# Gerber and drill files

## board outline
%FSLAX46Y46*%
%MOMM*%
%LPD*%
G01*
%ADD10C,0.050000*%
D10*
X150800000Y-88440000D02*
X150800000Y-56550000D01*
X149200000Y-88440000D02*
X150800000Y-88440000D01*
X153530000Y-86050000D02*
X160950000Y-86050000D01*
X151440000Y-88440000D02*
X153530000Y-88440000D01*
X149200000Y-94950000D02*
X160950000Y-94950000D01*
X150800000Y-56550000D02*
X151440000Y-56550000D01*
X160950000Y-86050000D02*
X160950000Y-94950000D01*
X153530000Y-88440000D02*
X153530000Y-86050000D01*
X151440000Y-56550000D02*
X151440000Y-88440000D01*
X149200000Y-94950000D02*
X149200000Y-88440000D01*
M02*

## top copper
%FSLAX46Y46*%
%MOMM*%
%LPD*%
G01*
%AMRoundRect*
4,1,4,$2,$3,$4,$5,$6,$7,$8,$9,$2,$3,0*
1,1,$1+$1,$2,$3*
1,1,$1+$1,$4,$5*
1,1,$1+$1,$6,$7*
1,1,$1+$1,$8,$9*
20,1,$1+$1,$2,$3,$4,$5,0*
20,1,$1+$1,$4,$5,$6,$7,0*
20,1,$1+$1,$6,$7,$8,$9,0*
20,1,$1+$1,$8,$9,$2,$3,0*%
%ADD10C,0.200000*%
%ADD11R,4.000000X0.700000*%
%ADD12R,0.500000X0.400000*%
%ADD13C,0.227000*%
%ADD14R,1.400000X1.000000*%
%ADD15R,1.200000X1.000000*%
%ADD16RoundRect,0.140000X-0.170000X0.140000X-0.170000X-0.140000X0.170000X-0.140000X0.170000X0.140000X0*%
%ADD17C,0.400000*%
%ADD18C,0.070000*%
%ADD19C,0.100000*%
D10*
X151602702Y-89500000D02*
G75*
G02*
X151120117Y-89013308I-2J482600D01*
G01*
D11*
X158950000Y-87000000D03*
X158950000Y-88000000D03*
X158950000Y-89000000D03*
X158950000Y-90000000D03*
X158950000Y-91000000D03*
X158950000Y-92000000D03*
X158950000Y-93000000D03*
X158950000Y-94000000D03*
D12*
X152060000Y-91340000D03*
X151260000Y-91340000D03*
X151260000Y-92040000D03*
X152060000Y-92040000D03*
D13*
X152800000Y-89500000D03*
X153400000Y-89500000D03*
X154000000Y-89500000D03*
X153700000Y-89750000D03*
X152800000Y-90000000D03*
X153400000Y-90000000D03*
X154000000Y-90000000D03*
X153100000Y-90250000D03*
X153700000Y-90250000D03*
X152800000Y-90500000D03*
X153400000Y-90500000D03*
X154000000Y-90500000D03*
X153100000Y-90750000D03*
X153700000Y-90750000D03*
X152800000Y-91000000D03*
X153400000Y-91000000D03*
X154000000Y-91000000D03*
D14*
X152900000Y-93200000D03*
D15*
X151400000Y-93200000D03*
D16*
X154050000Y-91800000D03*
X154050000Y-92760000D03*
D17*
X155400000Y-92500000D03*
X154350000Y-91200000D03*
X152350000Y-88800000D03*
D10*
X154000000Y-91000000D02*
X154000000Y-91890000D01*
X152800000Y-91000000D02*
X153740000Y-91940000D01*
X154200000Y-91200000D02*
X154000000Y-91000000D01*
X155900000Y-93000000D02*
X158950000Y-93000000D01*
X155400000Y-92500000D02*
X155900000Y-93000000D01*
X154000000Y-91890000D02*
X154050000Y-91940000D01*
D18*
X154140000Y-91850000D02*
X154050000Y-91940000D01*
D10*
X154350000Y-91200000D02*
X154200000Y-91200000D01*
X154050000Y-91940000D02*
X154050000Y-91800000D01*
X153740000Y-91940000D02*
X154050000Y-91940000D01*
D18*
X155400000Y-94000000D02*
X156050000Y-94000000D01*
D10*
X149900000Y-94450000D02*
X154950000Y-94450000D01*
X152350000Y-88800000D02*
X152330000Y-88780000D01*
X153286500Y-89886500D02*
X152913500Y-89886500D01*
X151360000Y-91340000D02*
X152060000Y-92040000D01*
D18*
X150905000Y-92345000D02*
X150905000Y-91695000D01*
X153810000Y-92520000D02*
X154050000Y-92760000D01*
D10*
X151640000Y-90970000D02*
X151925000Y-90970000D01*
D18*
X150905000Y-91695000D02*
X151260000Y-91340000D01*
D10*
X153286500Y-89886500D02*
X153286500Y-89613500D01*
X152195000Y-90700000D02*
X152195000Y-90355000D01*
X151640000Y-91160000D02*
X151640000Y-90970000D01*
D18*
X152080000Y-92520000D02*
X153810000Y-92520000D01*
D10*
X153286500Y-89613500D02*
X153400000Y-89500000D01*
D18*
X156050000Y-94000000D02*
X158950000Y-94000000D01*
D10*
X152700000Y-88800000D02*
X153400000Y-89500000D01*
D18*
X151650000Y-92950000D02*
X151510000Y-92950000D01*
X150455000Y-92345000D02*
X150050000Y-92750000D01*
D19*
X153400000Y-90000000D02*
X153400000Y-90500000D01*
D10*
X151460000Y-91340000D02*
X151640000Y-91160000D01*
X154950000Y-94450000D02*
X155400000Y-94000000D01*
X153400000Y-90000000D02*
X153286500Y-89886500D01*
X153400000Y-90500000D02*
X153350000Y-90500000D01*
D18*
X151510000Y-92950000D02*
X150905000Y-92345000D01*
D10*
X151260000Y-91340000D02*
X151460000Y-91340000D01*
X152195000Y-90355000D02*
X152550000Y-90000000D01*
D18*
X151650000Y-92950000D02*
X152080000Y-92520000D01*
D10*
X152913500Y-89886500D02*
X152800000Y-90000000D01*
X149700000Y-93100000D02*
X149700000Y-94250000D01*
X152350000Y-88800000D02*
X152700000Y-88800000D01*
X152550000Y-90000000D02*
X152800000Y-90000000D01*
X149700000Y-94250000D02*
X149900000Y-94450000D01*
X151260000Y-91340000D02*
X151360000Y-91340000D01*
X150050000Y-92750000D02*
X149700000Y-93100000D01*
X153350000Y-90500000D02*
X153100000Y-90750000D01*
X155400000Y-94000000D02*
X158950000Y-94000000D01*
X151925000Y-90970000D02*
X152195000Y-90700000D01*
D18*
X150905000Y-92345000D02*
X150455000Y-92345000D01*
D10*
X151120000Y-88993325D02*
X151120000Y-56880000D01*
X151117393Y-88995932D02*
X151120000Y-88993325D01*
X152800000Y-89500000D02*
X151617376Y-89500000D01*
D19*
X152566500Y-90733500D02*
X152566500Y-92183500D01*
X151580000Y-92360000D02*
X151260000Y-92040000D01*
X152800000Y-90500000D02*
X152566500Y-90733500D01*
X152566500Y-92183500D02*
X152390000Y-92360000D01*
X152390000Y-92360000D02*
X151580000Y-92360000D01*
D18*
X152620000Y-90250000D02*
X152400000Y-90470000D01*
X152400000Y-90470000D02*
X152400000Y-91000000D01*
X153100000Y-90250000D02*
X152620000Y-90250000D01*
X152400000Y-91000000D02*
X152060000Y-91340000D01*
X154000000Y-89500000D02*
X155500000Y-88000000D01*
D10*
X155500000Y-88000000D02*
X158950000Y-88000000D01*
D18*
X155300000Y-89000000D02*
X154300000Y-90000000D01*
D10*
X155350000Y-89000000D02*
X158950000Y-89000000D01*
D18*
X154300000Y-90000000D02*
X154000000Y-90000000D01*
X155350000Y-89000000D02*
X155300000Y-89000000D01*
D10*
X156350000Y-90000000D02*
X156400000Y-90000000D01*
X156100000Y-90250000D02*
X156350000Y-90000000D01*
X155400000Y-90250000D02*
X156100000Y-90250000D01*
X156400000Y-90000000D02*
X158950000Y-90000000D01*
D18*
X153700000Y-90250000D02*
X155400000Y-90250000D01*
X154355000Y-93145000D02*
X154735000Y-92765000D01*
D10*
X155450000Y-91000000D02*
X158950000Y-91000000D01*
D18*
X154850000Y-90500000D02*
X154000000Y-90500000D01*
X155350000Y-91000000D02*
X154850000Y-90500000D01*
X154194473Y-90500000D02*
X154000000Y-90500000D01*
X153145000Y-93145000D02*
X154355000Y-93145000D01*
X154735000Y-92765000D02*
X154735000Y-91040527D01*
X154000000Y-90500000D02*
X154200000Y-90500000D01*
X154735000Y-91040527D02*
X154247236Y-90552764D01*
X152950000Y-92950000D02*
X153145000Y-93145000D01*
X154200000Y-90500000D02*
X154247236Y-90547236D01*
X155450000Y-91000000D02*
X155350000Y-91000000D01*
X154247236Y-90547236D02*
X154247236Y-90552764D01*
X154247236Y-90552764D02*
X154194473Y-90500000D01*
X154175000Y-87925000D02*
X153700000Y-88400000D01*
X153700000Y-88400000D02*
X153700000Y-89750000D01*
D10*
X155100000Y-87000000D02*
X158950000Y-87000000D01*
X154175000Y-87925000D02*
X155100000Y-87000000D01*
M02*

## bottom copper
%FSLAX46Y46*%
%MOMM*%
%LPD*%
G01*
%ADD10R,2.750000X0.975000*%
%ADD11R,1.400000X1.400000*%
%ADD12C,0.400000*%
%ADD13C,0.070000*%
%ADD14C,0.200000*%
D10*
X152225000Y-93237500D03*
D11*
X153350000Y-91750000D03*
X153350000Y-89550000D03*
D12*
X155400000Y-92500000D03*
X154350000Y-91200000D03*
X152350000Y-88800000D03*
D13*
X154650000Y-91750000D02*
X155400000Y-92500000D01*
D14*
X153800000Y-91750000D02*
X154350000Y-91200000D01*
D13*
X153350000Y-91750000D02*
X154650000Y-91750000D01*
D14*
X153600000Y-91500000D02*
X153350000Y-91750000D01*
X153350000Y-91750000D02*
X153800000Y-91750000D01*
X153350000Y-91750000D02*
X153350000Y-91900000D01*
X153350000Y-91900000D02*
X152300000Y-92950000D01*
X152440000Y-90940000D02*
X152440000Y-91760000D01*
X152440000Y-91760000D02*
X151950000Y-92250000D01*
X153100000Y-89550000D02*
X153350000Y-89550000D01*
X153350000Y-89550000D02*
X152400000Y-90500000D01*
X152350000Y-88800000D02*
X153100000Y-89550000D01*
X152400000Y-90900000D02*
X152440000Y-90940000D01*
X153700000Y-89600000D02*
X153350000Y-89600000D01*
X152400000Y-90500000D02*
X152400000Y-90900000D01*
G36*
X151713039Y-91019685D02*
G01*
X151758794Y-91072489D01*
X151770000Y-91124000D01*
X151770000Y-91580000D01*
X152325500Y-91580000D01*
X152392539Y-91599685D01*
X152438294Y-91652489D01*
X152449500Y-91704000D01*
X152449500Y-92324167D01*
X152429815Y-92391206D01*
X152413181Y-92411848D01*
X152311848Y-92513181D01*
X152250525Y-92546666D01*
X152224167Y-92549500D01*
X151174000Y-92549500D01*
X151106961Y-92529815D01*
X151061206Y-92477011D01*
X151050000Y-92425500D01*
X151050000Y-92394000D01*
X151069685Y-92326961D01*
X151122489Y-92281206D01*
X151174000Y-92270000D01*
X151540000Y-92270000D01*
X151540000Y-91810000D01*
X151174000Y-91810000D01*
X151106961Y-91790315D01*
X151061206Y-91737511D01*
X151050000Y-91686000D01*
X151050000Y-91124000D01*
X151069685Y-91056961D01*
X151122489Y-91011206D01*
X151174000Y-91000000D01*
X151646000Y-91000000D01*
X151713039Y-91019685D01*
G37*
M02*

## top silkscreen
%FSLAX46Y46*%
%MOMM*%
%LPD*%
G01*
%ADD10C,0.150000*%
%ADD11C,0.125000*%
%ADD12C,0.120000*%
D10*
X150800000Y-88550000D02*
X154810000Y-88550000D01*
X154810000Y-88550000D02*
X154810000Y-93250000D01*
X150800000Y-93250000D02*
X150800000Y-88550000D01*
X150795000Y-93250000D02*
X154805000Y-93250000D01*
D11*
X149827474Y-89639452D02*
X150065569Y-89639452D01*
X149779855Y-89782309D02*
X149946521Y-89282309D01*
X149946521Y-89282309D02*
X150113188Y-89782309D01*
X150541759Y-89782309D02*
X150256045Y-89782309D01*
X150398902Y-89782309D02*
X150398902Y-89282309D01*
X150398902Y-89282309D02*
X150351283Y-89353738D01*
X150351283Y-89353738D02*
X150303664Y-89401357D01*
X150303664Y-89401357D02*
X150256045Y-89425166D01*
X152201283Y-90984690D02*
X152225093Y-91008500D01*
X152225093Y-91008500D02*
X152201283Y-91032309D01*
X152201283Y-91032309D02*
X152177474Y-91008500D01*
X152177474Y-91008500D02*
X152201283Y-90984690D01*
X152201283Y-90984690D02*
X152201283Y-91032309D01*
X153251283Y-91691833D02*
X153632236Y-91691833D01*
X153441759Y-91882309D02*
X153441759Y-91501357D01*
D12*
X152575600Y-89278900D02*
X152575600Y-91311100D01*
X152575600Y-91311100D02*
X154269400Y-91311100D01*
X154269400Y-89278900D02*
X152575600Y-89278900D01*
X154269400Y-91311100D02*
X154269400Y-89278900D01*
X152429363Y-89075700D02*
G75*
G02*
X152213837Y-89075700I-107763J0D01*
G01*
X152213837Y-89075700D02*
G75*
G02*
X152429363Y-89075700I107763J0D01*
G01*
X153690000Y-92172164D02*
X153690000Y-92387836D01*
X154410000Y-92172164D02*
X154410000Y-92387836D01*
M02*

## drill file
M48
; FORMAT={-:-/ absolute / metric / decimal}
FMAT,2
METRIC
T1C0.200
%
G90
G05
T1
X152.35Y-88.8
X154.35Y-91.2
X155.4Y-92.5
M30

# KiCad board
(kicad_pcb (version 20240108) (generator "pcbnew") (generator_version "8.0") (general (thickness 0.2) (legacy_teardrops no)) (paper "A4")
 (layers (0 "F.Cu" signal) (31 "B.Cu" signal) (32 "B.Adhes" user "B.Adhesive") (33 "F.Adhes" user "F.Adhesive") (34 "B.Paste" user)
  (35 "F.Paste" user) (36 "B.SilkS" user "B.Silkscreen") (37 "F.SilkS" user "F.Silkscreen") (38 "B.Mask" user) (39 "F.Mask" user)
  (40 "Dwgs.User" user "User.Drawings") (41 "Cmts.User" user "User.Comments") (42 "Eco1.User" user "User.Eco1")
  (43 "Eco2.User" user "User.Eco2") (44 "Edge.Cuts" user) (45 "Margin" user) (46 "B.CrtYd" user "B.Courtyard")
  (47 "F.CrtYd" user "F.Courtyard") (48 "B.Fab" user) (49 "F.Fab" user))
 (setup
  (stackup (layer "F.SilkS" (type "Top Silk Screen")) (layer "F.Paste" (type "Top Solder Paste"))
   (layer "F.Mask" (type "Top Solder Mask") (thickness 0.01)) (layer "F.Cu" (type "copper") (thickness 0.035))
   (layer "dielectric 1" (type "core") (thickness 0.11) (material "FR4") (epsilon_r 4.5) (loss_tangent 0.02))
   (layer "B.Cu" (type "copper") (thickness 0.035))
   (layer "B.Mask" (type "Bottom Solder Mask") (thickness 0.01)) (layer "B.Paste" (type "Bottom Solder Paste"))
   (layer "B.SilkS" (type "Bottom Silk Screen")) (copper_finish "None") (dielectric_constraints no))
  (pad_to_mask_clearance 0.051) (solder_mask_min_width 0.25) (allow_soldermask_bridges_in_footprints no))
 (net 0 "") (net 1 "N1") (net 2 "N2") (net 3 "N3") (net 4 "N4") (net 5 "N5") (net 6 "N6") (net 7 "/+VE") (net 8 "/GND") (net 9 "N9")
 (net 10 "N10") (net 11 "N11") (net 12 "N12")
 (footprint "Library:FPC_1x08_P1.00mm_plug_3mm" (layer "F.Cu") (at 156.95 90.5)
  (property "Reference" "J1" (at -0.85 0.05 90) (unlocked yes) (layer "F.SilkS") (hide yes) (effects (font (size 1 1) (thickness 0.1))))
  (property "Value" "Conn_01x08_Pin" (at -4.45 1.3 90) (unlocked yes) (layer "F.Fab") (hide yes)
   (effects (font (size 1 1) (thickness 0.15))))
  (pad "1" connect rect (at 2 -3.5) (size 4 0.7) (layers "F.Cu" "F.Mask") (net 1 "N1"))
  (pad "2" connect rect (at 2 -2.5) (size 4 0.7) (layers "F.Cu" "F.Mask") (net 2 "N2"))
  (pad "3" connect rect (at 2 -1.5) (size 4 0.7) (layers "F.Cu" "F.Mask") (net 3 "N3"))
  (pad "4" connect rect (at 2 -0.5) (size 4 0.7) (layers "F.Cu" "F.Mask") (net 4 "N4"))
  (pad "5" connect rect (at 2 0.5) (size 4 0.7) (layers "F.Cu" "F.Mask") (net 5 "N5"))
  (pad "6" connect rect (at 2 1.5) (size 4 0.7) (layers "F.Cu" "F.Mask") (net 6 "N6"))
  (pad "7" connect rect (at 2 2.5) (size 4 0.7) (layers "F.Cu" "F.Mask") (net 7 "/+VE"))
  (pad "8" connect rect (at 2 3.5) (size 4 0.7) (layers "F.Cu" "F.Mask") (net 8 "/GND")))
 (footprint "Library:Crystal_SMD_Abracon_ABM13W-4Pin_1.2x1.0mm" (layer "F.Cu") (at 151.66 91.69 180)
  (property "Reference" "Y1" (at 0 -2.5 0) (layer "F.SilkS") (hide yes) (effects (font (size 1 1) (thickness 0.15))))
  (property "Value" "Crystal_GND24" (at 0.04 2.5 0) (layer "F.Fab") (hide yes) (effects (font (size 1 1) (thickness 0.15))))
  (pad "1" smd rect (at -0.4 0.35 180) (size 0.5 0.4) (layers "F.Cu" "F.Paste" "F.Mask") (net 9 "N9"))
  (pad "2" smd rect (at 0.4 0.35 180) (size 0.5 0.4) (layers "F.Cu" "F.Paste" "F.Mask") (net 8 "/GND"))
  (pad "3" smd rect (at 0.4 -0.35 180) (size 0.5 0.4) (layers "F.Cu" "F.Paste" "F.Mask") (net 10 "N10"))
  (pad "4" smd rect (at -0.4 -0.35 180) (size 0.5 0.4) (layers "F.Cu" "F.Paste" "F.Mask") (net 8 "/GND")))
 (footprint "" (layer "F.Cu") (at 152.1 93.35)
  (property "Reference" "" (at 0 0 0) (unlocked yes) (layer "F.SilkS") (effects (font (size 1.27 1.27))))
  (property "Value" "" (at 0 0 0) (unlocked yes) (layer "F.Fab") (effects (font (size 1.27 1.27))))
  (pad "2" smd rect (at 0.125 -0.1125 270) (size 0.975 2.75) (layers "B.Cu" "B.Paste" "B.Mask") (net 7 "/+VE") (solder_mask_margin 0.102)))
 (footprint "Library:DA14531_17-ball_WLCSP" (layer "F.Cu") (at 153.422 90.295)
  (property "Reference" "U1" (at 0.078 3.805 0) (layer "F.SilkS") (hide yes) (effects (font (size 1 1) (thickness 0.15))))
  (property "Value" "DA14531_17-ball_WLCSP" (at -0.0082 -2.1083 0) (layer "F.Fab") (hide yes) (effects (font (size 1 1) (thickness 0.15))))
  (fp_line (start -0.8464 -1.0161) (end -0.8464 1.0161) (stroke (width 0.12) (type solid)) (layer "F.SilkS"))
  (fp_line (start -0.8464 1.0161) (end 0.8474 1.0161) (stroke (width 0.12) (type solid)) (layer "F.SilkS"))
  (fp_line (start 0.8474 -1.0161) (end -0.8464 -1.0161) (stroke (width 0.12) (type solid)) (layer "F.SilkS"))
  (fp_line (start 0.8474 1.0161) (end 0.8474 -1.0161) (stroke (width 0.12) (type solid)) (layer "F.SilkS"))
  (fp_circle (center -1.1004 -1.2193) (end -1.0242 -1.1431) (stroke (width 0.12) (type solid)) (fill none) (layer "F.SilkS"))
  (pad "A1" smd circle (at -0.622 -0.795) (size 0.227 0.227) (layers "F.Cu" "F.Paste" "F.Mask") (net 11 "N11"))
  (pad "A3" smd circle (at -0.022 -0.795) (size 0.227 0.227) (layers "F.Cu" "F.Paste" "F.Mask") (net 8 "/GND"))
  (pad "A5" smd circle (at 0.578 -0.795) (size 0.227 0.227) (layers "F.Cu" "F.Paste" "F.Mask") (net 2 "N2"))
  (pad "B4" smd circle (at 0.278 -0.545) (size 0.227 0.227) (layers "F.Cu" "F.Paste" "F.Mask") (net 1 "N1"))
  (pad "C1" smd circle (at -0.622 -0.295) (size 0.227 0.227) (layers "F.Cu" "F.Paste" "F.Mask") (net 8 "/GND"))
  (pad "C3" smd circle (at -0.022 -0.295) (size 0.227 0.227) (layers "F.Cu" "F.Paste" "F.Mask") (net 8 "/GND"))
  (pad "C5" smd circle (at 0.578 -0.295) (size 0.227 0.227) (layers "F.Cu" "F.Paste" "F.Mask") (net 3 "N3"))
  (pad "D2" smd circle (at -0.322 -0.045) (size 0.227 0.227) (layers "F.Cu" "F.Paste" "F.Mask") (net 9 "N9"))
  (pad "D4" smd circle (at 0.278 -0.045) (size 0.227 0.227) (layers "F.Cu" "F.Paste" "F.Mask") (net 4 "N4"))
  (pad "E1" smd circle (at -0.622 0.205) (size 0.227 0.227) (layers "F.Cu" "F.Paste" "F.Mask") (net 10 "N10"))
  (pad "E3" smd circle (at -0.022 0.205) (size 0.227 0.227) (layers "F.Cu" "F.Paste" "F.Mask") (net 8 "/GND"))
  (pad "E5" smd circle (at 0.578 0.205) (size 0.227 0.227) (layers "F.Cu" "F.Paste" "F.Mask") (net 5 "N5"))
  (pad "F2" smd circle (at -0.322 0.455) (size 0.227 0.227) (layers "F.Cu" "F.Paste" "F.Mask") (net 8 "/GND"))
  (pad "F4" smd circle (at 0.278 0.455) (size 0.227 0.227) (layers "F.Cu" "F.Paste" "F.Mask") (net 6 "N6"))
  (pad "G1" smd circle (at -0.622 0.705) (size 0.227 0.227) (layers "F.Cu" "F.Paste" "F.Mask") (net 7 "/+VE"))
  (pad "G3" smd circle (at -0.022 0.705) (size 0.227 0.227) (layers "F.Cu" "F.Paste" "F.Mask") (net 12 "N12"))
  (pad "G5" smd circle (at 0.578 0.705) (size 0.227 0.227) (layers "F.Cu" "F.Paste" "F.Mask") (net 7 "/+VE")))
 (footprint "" (layer "F.Cu") (at 152.9 93.3)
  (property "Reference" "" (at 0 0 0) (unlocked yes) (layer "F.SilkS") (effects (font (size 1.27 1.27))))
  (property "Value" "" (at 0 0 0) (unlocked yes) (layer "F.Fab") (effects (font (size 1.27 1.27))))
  (pad "2" smd rect (at 0 -0.1 270) (size 1 1.4) (layers "F.Cu" "F.Paste" "F.Mask") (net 5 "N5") (solder_mask_margin 0.102)))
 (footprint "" (layer "F.Cu") (at 151.3 93.3)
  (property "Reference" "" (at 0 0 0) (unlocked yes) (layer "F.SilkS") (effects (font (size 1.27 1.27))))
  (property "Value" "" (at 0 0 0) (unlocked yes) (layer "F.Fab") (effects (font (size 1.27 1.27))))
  (pad "2" smd rect (at 0.1 -0.1 270) (size 1 1.2) (layers "F.Cu" "F.Paste" "F.Mask") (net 8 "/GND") (solder_mask_margin 0.102)))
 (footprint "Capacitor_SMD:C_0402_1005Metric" (layer "F.Cu") (at 154.05 92.28 -90)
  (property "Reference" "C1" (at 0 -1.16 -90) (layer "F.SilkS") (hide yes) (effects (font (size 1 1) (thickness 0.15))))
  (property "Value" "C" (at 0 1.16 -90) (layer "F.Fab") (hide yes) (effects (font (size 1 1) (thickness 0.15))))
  (fp_line (start -0.107836 0.36) (end 0.107836 0.36) (stroke (width 0.12) (type solid)) (layer "F.SilkS"))
  (fp_line (start -0.107836 -0.36) (end 0.107836 -0.36) (stroke (width 0.12) (type solid)) (layer "F.SilkS"))
  (pad "1" smd roundrect (at -0.48 0 270) (size 0.56 0.62) (layers "F.Cu" "F.Paste" "F.Mask") (roundrect_rratio 0.25) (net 7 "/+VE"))
  (pad "2" smd roundrect (at 0.48 0 270) (size 0.56 0.62) (layers "F.Cu" "F.Paste" "F.Mask") (roundrect_rratio 0.25) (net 8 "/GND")))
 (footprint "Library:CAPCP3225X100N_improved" (layer "B.Cu") (at 153.35 90.65 90)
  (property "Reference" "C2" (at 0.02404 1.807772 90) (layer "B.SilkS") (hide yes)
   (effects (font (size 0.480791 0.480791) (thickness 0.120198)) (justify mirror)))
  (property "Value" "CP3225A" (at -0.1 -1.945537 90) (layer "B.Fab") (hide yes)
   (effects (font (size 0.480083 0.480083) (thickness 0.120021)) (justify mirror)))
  (pad "1" smd rect (at -1.1 0 270) (size 1.4 1.4) (layers "B.Cu" "B.Paste" "B.Mask") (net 7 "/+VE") (solder_mask_margin 0.102))
  (pad "2" smd rect (at 1.1 0 270) (size 1.4 1.4) (layers "B.Cu" "B.Paste" "B.Mask") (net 8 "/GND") (solder_mask_margin 0.102)))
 (gr_arc (start 151.602702 89.5) (mid 151.26 89.357201) (end 151.120095 89.013308) (stroke (width 0.2) (type default)) (layer "F.Cu")
  (net 11))
 (gr_line (start 150.8 88.55) (end 154.81 88.55) (stroke (width 0.15) (type default)) (layer "F.SilkS"))
 (gr_line (start 154.81 88.55) (end 154.81 93.25) (stroke (width 0.15) (type default)) (layer "F.SilkS"))
 (gr_line (start 150.8 93.25) (end 150.8 88.55) (stroke (width 0.15) (type default)) (layer "F.SilkS"))
 (gr_line (start 150.795 93.25) (end 154.805 93.25) (stroke (width 0.15) (type default)) (layer "F.SilkS"))
 (gr_line (start 150.8 88.44) (end 150.8 56.55) (stroke (width 0.05) (type default)) (layer "Edge.Cuts"))
 (gr_line (start 149.2 88.44) (end 150.8 88.44) (stroke (width 0.05) (type default)) (layer "Edge.Cuts"))
 (gr_line (start 153.53 86.05) (end 160.95 86.05) (stroke (width 0.05) (type default)) (layer "Edge.Cuts"))
 (gr_line (start 151.44 88.44) (end 153.53 88.44) (stroke (width 0.05) (type default)) (layer "Edge.Cuts"))
 (gr_line (start 149.2 94.95) (end 160.95 94.95) (stroke (width 0.05) (type default)) (layer "Edge.Cuts"))
 (gr_line (start 150.8 56.55) (end 151.44 56.55) (stroke (width 0.05) (type default)) (layer "Edge.Cuts"))
 (gr_line (start 160.95 86.05) (end 160.95 94.95) (stroke (width 0.05) (type default)) (layer "Edge.Cuts"))
 (gr_line (start 153.53 88.44) (end 153.53 86.05) (stroke (width 0.05) (type default)) (layer "Edge.Cuts"))
 (gr_line (start 151.44 56.55) (end 151.44 88.44) (stroke (width 0.05) (type default)) (layer "Edge.Cuts"))
 (gr_line (start 149.2 94.95) (end 149.2 88.44) (stroke (width 0.05) (type default)) (layer "Edge.Cuts"))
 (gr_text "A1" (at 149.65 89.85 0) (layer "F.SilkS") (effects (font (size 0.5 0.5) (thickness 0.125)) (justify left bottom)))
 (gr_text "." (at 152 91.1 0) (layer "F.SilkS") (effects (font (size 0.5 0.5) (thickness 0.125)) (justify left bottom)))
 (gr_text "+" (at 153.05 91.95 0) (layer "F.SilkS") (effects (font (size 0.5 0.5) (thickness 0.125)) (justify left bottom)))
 (segment (start 154 91) (end 154 91.89) (width 0.2) (layer "F.Cu") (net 7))
 (segment (start 152.8 91) (end 153.74 91.94) (width 0.2) (layer "F.Cu") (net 7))
 (segment (start 154.2 91.2) (end 154 91) (width 0.2) (layer "F.Cu") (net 7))
 (segment (start 155.9 93) (end 158.95 93) (width 0.2) (layer "F.Cu") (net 7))
 (segment (start 155.4 92.5) (end 155.9 93) (width 0.2) (layer "F.Cu") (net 7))
 (segment (start 154 91.89) (end 154.05 91.94) (width 0.2) (layer "F.Cu") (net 7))
 (segment (start 154.14 91.85) (end 154.05 91.94) (width 0.07) (layer "F.Cu") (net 7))
 (segment (start 154.35 91.2) (end 154.2 91.2) (width 0.2) (layer "F.Cu") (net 7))
 (segment (start 154.05 91.94) (end 154.05 91.8) (width 0.2) (layer "F.Cu") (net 7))
 (segment (start 153.74 91.94) (end 154.05 91.94) (width 0.2) (layer "F.Cu") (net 7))
 (via (at 155.4 92.5) (size 0.4) (drill 0.2) (layers "F.Cu" "B.Cu") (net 7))
 (via (at 154.35 91.2) (size 0.4) (drill 0.2) (layers "F.Cu" "B.Cu") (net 7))
 (segment (start 154.65 91.75) (end 155.4 92.5) (width 0.07) (layer "B.Cu") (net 7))
 (segment (start 153.8 91.75) (end 154.35 91.2) (width 0.2) (layer "B.Cu") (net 7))
 (segment (start 153.35 91.75) (end 154.65 91.75) (width 0.07) (layer "B.Cu") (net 7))
 (segment (start 153.6 91.5) (end 153.35 91.75) (width 0.2) (layer "B.Cu") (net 7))
 (segment (start 153.35 91.75) (end 153.8 91.75) (width 0.2) (layer "B.Cu") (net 7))
 (segment (start 153.35 91.75) (end 153.35 91.9) (width 0.2) (layer "B.Cu") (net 7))
 (segment (start 153.35 91.9) (end 152.3 92.95) (width 0.2) (layer "B.Cu") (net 7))
 (segment (start 155.4 94) (end 156.05 94) (width 0.07) (layer "F.Cu") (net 8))
 (segment (start 149.9 94.45) (end 154.95 94.45) (width 0.2) (layer "F.Cu") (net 8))
 (segment (start 152.35 88.8) (end 152.33 88.78) (width 0.2) (layer "F.Cu") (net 8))
 (segment (start 153.2865 89.8865) (end 152.9135 89.8865) (width 0.2) (layer "F.Cu") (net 8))
 (segment (start 151.36 91.34) (end 152.06 92.04) (width 0.2) (layer "F.Cu") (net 8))
 (segment (start 150.905 92.345) (end 150.905 91.695) (width 0.07) (layer "F.Cu") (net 8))
 (segment (start 153.81 92.52) (end 154.05 92.76) (width 0.07) (layer "F.Cu") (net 8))
 (segment (start 151.64 90.97) (end 151.925 90.97) (width 0.2) (layer "F.Cu") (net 8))
 (segment (start 150.905 91.695) (end 151.26 91.34) (width 0.07) (layer "F.Cu") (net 8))
 (segment (start 153.2865 89.8865) (end 153.2865 89.6135) (width 0.2) (layer "F.Cu") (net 8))
 (segment (start 152.195 90.7) (end 152.195 90.355) (width 0.2) (layer "F.Cu") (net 8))
 (segment (start 151.64 91.16) (end 151.64 90.97) (width 0.2) (layer "F.Cu") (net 8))
 (segment (start 152.08 92.52) (end 153.81 92.52) (width 0.07) (layer "F.Cu") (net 8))
 (segment (start 153.2865 89.6135) (end 153.4 89.5) (width 0.2) (layer "F.Cu") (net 8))
 (segment (start 156.05 94) (end 158.95 94) (width 0.07) (layer "F.Cu") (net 8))
 (segment (start 152.7 88.8) (end 153.4 89.5) (width 0.2) (layer "F.Cu") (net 8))
 (segment (start 151.65 92.95) (end 151.51 92.95) (width 0.07) (layer "F.Cu") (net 8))
 (segment (start 150.455 92.345) (end 150.05 92.75) (width 0.07) (layer "F.Cu") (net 8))
 (segment (start 153.4 90) (end 153.4 90.5) (width 0.1) (layer "F.Cu") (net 8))
 (segment (start 151.46 91.34) (end 151.64 91.16) (width 0.2) (layer "F.Cu") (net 8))
 (segment (start 154.95 94.45) (end 155.4 94) (width 0.2) (layer "F.Cu") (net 8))
 (segment (start 153.4 90) (end 153.2865 89.8865) (width 0.2) (layer "F.Cu") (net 8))
 (segment (start 153.4 90.5) (end 153.35 90.5) (width 0.2) (layer "F.Cu") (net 8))
 (segment (start 151.51 92.95) (end 150.905 92.345) (width 0.07) (layer "F.Cu") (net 8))
 (segment (start 151.26 91.34) (end 151.46 91.34) (width 0.2) (layer "F.Cu") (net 8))
 (segment (start 152.195 90.355) (end 152.55 90) (width 0.2) (layer "F.Cu") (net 8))
 (segment (start 151.65 92.95) (end 152.08 92.52) (width 0.07) (layer "F.Cu") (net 8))
 (segment (start 152.9135 89.8865) (end 152.8 90) (width 0.2) (layer "F.Cu") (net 8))
 (segment (start 149.7 93.1) (end 149.7 94.25) (width 0.2) (layer "F.Cu") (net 8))
 (segment (start 152.35 88.8) (end 152.7 88.8) (width 0.2) (layer "F.Cu") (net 8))
 (segment (start 152.55 90) (end 152.8 90) (width 0.2) (layer "F.Cu") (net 8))
 (segment (start 149.7 94.25) (end 149.9 94.45) (width 0.2) (layer "F.Cu") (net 8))
 (segment (start 151.26 91.34) (end 151.36 91.34) (width 0.2) (layer "F.Cu") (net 8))
 (segment (start 150.05 92.75) (end 149.7 93.1) (width 0.2) (layer "F.Cu") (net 8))
 (segment (start 153.35 90.5) (end 153.1 90.75) (width 0.2) (layer "F.Cu") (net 8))
 (segment (start 155.4 94) (end 158.95 94) (width 0.2) (layer "F.Cu") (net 8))
 (segment (start 151.925 90.97) (end 152.195 90.7) (width 0.2) (layer "F.Cu") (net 8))
 (segment (start 150.905 92.345) (end 150.455 92.345) (width 0.07) (layer "F.Cu") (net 8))
 (via (at 152.35 88.8) (size 0.4) (drill 0.2) (layers "F.Cu" "B.Cu") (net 8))
 (segment (start 152.44 90.94) (end 152.44 91.76) (width 0.2) (layer "B.Cu") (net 8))
 (segment (start 152.44 91.76) (end 151.95 92.25) (width 0.2) (layer "B.Cu") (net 8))
 (segment (start 153.1 89.55) (end 153.35 89.55) (width 0.2) (layer "B.Cu") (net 8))
 (segment (start 153.35 89.55) (end 152.4 90.5) (width 0.2) (layer "B.Cu") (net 8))
 (segment (start 152.35 88.8) (end 153.1 89.55) (width 0.2) (layer "B.Cu") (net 8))
 (segment (start 152.4 90.9) (end 152.44 90.94) (width 0.2) (layer "B.Cu") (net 8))
 (segment (start 153.7 89.6) (end 153.35 89.6) (width 0.2) (layer "B.Cu") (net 8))
 (segment (start 152.4 90.5) (end 152.4 90.9) (width 0.2) (layer "B.Cu") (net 8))
 (segment (start 151.12 88.993325) (end 151.12 56.88) (width 0.2) (layer "F.Cu") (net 11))
 (segment (start 151.117393 88.995932) (end 151.12 88.993325) (width 0.2) (layer "F.Cu") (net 11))
 (segment (start 152.8 89.5) (end 151.617376 89.5) (width 0.2) (layer "F.Cu") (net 11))
 (segment (start 152.5665 90.7335) (end 152.5665 92.1835) (width 0.1) (layer "F.Cu") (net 10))
 (segment (start 151.58 92.36) (end 151.26 92.04) (width 0.1) (layer "F.Cu") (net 10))
 (segment (start 152.8 90.5) (end 152.5665 90.7335) (width 0.1) (layer "F.Cu") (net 10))
 (segment (start 152.5665 92.1835) (end 152.39 92.36) (width 0.1) (layer "F.Cu") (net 10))
 (segment (start 152.39 92.36) (end 151.58 92.36) (width 0.1) (layer "F.Cu") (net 10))
 (segment (start 152.62 90.25) (end 152.4 90.47) (width 0.07) (layer "F.Cu") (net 9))
 (segment (start 152.4 90.47) (end 152.4 91) (width 0.07) (layer "F.Cu") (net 9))
 (segment (start 153.1 90.25) (end 152.62 90.25) (width 0.07) (layer "F.Cu") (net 9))
 (segment (start 152.4 91) (end 152.06 91.34) (width 0.07) (layer "F.Cu") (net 9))
 (segment (start 154 89.5) (end 155.5 88) (width 0.07) (layer "F.Cu") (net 2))
 (segment (start 155.5 88) (end 158.95 88) (width 0.2) (layer "F.Cu") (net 2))
 (segment (start 155.3 89) (end 154.3 90) (width 0.07) (layer "F.Cu") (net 3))
 (segment (start 155.35 89) (end 158.95 89) (width 0.2) (layer "F.Cu") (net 3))
 (segment (start 154.3 90) (end 154 90) (width 0.07) (layer "F.Cu") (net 3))
 (segment (start 155.35 89) (end 155.3 89) (width 0.07) (layer "F.Cu") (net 3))
 (segment (start 156.35 90) (end 156.4 90) (width 0.2) (layer "F.Cu") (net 4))
 (segment (start 156.1 90.25) (end 156.35 90) (width 0.2) (layer "F.Cu") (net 4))
 (segment (start 155.4 90.25) (end 156.1 90.25) (width 0.2) (layer "F.Cu") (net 4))
 (segment (start 156.4 90) (end 158.95 90) (width 0.2) (layer "F.Cu") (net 4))
 (segment (start 153.7 90.25) (end 155.4 90.25) (width 0.07) (layer "F.Cu") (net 4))
 (segment (start 154.355 93.145) (end 154.735 92.765) (width 0.07) (layer "F.Cu") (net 5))
 (segment (start 155.45 91) (end 158.95 91) (width 0.2) (layer "F.Cu") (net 5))
 (segment (start 154.85 90.5) (end 154 90.5) (width 0.07) (layer "F.Cu") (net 5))
 (segment (start 155.35 91) (end 154.85 90.5) (width 0.07) (layer "F.Cu") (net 5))
 (segment (start 154.194473 90.5) (end 154 90.5) (width 0.07) (layer "F.Cu") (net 5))
 (segment (start 153.145 93.145) (end 154.355 93.145) (width 0.07) (layer "F.Cu") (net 5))
 (segment (start 154.735 92.765) (end 154.735 91.040527) (width 0.07) (layer "F.Cu") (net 5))
 (segment (start 154 90.5) (end 154.2 90.5) (width 0.07) (layer "F.Cu") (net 5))
 (segment (start 154.735 91.040527) (end 154.247236 90.552764) (width 0.07) (layer "F.Cu") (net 5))
 (segment (start 152.95 92.95) (end 153.145 93.145) (width 0.07) (layer "F.Cu") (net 5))
 (segment (start 154.2 90.5) (end 154.247236 90.547236) (width 0.07) (layer "F.Cu") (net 5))
 (segment (start 155.45 91) (end 155.35 91) (width 0.07) (layer "F.Cu") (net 5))
 (segment (start 154.247236 90.547236) (end 154.247236 90.552764) (width 0.07) (layer "F.Cu") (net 5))
 (segment (start 154.247236 90.552764) (end 154.194473 90.5) (width 0.07) (layer "F.Cu") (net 5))
 (segment (start 154.175 87.925) (end 153.7 88.4) (width 0.07) (layer "F.Cu") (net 1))
 (segment (start 153.7 88.4) (end 153.7 89.75) (width 0.07) (layer "F.Cu") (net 1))
 (segment (start 155.1 87) (end 158.95 87) (width 0.2) (layer "F.Cu") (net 1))
 (segment (start 154.175 87.925) (end 155.1 87) (width 0.2) (layer "F.Cu") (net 1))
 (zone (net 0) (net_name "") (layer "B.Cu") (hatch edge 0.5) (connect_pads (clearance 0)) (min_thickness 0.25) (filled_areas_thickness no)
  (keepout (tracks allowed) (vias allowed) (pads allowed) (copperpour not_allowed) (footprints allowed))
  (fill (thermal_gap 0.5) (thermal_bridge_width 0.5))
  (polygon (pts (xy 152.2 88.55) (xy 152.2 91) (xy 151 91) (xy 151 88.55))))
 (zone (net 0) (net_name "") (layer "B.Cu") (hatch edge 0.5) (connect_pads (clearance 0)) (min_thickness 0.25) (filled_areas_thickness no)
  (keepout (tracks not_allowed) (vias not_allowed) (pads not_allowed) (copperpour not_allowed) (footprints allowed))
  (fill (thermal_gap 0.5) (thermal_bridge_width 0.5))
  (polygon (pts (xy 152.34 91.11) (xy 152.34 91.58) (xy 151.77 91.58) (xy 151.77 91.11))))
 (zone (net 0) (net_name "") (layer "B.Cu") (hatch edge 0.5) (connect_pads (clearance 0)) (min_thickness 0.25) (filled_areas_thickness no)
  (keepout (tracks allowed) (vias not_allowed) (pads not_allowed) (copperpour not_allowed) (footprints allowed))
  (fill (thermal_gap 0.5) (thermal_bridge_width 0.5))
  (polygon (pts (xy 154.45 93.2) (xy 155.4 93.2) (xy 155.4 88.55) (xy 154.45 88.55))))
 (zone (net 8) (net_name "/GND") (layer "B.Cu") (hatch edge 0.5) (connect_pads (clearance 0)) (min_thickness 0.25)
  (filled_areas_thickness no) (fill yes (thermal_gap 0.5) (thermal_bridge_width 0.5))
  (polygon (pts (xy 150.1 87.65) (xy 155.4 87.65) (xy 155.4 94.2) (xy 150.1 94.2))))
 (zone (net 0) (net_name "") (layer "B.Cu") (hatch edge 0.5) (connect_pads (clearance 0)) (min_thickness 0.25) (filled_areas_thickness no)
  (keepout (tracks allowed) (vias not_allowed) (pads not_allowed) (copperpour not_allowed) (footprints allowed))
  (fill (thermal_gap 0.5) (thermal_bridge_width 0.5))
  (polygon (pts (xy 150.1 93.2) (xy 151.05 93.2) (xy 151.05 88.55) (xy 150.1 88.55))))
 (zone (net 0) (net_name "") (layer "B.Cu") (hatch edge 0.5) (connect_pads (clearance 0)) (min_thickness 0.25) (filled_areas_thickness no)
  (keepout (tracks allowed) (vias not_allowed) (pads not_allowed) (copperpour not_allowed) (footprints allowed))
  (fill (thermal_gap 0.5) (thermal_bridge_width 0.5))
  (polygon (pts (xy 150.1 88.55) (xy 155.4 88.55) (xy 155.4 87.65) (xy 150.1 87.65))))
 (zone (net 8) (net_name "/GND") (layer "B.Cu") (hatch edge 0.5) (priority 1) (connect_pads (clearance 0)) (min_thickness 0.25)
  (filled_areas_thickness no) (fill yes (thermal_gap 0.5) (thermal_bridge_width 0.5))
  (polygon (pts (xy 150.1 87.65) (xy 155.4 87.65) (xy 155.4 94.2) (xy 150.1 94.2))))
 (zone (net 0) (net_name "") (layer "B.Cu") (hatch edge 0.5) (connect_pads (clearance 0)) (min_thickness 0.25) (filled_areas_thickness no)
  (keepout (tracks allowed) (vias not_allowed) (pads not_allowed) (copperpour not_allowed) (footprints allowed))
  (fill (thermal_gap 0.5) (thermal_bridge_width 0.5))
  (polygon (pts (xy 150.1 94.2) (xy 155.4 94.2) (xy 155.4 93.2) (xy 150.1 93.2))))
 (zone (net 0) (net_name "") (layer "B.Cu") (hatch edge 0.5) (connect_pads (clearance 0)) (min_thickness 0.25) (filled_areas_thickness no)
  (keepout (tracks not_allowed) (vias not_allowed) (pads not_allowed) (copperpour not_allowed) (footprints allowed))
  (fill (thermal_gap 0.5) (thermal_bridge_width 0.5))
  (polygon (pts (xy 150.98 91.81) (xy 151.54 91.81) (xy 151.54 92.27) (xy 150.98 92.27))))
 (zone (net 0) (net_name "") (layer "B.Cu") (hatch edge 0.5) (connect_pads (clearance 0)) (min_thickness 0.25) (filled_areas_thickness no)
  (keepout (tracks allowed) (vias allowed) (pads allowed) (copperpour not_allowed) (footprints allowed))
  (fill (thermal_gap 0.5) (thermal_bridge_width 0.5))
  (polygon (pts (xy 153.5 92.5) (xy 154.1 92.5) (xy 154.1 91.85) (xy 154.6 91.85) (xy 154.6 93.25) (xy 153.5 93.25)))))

